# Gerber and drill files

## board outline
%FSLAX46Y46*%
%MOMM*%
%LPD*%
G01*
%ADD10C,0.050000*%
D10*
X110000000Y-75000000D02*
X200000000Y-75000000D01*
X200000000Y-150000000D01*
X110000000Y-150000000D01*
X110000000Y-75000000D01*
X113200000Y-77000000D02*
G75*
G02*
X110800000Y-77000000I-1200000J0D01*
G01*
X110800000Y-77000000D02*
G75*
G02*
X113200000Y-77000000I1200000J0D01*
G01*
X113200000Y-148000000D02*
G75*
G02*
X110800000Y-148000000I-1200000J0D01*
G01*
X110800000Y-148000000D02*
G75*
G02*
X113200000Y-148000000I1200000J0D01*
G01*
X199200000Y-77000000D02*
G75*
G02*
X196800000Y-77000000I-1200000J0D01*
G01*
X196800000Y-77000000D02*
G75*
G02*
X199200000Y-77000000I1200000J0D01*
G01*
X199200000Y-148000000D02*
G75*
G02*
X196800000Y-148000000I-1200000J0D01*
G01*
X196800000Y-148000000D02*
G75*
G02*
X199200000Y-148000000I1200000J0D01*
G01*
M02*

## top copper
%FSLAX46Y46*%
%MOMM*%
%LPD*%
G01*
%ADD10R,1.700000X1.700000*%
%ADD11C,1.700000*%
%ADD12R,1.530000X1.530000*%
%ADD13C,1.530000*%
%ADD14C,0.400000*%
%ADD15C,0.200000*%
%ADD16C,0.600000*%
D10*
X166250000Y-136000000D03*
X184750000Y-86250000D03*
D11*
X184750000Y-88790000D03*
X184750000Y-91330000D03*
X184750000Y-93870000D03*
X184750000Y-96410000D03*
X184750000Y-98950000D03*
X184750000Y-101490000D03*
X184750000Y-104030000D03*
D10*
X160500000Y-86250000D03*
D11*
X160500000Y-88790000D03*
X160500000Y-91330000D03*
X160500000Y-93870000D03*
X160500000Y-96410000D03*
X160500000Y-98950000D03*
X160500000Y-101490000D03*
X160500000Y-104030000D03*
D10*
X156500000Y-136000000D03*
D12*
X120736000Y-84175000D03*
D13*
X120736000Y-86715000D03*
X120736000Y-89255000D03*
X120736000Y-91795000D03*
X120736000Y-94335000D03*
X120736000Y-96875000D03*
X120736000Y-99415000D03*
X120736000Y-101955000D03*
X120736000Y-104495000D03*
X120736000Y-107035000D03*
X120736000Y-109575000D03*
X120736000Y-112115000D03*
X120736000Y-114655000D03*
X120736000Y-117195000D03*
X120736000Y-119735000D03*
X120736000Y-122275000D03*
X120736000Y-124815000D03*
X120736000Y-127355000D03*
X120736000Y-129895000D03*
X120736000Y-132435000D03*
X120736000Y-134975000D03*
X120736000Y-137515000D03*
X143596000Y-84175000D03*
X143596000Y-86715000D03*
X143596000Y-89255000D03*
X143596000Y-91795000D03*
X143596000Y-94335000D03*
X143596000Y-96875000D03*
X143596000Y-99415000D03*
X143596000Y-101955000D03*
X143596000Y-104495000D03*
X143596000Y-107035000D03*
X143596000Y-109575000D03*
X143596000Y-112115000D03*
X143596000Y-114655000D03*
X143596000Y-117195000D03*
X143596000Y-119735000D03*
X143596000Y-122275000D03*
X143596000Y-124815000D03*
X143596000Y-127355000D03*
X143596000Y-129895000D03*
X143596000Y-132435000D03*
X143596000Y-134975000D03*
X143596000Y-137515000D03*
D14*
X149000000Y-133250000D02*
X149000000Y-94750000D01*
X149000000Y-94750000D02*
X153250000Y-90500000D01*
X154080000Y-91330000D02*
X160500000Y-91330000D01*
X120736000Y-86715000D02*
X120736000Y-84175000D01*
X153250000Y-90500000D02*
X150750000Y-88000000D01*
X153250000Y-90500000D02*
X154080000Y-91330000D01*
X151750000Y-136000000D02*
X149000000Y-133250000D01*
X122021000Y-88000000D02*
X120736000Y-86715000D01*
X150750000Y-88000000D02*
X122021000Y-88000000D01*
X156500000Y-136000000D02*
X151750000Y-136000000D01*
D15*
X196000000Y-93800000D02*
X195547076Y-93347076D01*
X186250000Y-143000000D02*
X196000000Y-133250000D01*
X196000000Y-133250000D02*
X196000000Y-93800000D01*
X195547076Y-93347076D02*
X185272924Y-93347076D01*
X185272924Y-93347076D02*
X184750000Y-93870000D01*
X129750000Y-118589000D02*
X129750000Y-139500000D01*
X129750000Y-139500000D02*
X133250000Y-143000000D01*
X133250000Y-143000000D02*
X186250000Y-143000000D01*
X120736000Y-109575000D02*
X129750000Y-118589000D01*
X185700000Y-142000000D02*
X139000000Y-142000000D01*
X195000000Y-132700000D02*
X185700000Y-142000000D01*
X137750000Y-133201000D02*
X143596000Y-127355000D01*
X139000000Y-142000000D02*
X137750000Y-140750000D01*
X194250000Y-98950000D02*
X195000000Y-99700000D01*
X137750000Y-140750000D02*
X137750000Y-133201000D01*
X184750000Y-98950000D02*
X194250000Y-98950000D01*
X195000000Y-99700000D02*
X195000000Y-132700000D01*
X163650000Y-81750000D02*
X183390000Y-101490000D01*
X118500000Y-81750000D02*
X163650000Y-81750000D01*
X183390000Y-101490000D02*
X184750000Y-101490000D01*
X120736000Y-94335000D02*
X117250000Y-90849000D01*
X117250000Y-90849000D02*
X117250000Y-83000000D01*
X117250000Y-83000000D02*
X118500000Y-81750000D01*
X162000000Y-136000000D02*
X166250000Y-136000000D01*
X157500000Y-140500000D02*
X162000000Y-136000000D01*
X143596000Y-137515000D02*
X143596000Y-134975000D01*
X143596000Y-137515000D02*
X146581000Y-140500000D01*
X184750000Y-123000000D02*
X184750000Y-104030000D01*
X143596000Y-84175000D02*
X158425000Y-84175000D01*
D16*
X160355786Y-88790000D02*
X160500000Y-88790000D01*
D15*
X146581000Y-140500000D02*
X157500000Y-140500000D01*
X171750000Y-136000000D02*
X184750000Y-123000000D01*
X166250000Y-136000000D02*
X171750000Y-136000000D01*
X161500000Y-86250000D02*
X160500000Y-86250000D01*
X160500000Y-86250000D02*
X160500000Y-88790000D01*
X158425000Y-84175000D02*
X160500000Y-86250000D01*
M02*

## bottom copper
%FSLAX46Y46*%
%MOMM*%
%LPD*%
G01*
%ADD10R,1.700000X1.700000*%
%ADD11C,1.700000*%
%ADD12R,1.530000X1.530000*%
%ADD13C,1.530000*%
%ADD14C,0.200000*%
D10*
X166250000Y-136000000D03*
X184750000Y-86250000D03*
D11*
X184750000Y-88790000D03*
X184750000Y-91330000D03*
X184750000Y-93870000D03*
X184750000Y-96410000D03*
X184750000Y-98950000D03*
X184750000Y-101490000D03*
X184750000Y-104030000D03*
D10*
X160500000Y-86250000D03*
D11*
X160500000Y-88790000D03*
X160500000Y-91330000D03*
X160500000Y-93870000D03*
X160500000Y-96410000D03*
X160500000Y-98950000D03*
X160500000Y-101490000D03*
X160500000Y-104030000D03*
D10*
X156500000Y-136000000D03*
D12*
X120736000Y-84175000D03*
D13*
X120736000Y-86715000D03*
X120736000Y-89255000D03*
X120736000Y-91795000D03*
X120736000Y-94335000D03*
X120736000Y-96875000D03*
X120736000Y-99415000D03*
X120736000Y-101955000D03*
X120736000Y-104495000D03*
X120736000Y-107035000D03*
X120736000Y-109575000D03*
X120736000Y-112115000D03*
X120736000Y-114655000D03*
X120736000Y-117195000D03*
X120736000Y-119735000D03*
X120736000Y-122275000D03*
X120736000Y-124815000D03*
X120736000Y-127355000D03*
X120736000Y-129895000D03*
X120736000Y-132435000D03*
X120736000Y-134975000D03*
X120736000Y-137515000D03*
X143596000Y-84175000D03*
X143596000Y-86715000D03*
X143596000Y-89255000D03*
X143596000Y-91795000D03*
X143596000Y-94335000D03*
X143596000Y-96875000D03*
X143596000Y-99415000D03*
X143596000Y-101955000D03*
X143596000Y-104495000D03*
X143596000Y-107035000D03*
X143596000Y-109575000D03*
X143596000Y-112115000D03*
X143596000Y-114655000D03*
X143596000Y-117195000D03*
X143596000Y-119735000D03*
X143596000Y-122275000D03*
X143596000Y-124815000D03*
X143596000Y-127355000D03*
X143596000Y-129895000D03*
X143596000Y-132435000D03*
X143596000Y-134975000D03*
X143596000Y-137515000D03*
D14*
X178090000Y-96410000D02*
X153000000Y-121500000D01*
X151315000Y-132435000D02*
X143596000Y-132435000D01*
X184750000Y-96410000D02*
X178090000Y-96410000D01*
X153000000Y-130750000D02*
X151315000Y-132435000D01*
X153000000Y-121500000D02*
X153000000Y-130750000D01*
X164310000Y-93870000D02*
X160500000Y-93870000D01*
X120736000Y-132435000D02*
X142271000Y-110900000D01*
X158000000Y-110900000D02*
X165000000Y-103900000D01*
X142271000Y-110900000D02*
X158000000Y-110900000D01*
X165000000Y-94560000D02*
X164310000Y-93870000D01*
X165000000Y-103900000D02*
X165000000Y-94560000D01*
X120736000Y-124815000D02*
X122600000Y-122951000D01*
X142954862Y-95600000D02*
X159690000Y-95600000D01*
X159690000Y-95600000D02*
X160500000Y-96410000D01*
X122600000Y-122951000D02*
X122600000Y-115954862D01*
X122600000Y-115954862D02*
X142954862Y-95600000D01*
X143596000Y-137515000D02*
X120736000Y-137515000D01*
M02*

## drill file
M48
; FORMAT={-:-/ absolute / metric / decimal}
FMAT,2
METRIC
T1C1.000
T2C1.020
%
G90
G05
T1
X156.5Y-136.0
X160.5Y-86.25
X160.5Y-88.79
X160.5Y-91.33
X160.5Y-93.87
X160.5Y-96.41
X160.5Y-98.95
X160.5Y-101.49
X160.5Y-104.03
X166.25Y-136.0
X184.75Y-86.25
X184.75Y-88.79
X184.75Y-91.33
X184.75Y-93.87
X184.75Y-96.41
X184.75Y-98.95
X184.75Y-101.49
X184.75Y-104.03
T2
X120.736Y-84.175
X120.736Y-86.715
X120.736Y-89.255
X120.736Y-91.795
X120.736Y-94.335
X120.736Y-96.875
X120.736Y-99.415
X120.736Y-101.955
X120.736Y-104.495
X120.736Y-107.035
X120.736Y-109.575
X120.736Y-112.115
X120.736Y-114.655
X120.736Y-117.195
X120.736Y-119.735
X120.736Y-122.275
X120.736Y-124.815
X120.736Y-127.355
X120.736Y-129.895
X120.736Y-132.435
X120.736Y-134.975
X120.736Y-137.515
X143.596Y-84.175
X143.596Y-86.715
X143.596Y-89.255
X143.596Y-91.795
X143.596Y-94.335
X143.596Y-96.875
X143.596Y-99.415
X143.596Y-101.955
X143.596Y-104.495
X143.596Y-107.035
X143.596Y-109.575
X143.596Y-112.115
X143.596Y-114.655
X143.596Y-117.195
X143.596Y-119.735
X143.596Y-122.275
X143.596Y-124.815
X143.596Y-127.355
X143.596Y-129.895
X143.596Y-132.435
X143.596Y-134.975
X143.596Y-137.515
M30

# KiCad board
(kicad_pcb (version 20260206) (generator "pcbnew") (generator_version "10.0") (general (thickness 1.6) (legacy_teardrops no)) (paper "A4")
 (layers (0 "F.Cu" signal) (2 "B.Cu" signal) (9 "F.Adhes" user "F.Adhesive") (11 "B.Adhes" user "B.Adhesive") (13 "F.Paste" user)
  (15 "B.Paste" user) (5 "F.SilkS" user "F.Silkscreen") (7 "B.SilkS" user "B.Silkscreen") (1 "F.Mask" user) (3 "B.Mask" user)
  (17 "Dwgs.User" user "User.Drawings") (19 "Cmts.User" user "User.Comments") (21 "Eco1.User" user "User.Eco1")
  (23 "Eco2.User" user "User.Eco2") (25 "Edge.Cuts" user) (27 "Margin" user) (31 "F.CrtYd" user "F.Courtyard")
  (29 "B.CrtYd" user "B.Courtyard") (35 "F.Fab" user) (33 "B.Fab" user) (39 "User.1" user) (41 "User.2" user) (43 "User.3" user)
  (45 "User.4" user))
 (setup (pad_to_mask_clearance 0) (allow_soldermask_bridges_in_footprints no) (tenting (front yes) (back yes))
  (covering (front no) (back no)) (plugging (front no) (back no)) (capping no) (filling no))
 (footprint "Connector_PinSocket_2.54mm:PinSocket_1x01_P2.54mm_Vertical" (layer "F.Cu") (at 166.25 136 180)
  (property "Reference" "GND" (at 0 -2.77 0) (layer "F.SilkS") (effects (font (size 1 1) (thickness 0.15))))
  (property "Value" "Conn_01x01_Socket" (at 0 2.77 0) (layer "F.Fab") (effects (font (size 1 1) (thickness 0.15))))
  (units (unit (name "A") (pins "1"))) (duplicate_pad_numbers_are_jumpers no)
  (pad "1" thru_hole rect (at 0 0 180) (size 1.7 1.7) (drill 1) (layers "*.Cu" "*.Mask") (remove_unused_layers no) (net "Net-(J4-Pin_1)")))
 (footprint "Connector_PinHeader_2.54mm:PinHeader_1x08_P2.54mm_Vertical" (layer "F.Cu") (at 184.75 86.25)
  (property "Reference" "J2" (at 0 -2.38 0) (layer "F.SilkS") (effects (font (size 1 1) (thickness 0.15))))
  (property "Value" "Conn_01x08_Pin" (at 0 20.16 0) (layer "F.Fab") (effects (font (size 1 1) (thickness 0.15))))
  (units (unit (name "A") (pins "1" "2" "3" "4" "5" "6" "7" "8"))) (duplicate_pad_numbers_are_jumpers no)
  (pad "1" thru_hole rect (at 0 0) (size 1.7 1.7) (drill 1) (layers "*.Cu" "*.Mask") (remove_unused_layers no)
   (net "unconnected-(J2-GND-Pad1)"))
  (pad "2" thru_hole circle (at 0 2.54) (size 1.7 1.7) (drill 1) (layers "*.Cu" "*.Mask") (remove_unused_layers no)
   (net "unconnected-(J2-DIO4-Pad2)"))
  (pad "3" thru_hole circle (at 0 5.08) (size 1.7 1.7) (drill 1) (layers "*.Cu" "*.Mask") (remove_unused_layers no)
   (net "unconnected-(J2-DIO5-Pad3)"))
  (pad "4" thru_hole circle (at 0 7.62) (size 1.7 1.7) (drill 1) (layers "*.Cu" "*.Mask") (remove_unused_layers no) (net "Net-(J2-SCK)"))
  (pad "5" thru_hole circle (at 0 10.16) (size 1.7 1.7) (drill 1) (layers "*.Cu" "*.Mask") (remove_unused_layers no) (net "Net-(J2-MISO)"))
  (pad "6" thru_hole circle (at 0 12.7) (size 1.7 1.7) (drill 1) (layers "*.Cu" "*.Mask") (remove_unused_layers no) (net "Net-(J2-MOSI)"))
  (pad "7" thru_hole circle (at 0 15.24) (size 1.7 1.7) (drill 1) (layers "*.Cu" "*.Mask") (remove_unused_layers no) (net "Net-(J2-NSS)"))
  (pad "8" thru_hole circle (at 0 17.78) (size 1.7 1.7) (drill 1) (layers "*.Cu" "*.Mask") (remove_unused_layers no) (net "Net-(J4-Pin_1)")))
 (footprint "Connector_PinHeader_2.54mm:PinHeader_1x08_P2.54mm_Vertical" (layer "F.Cu") (at 160.5 86.25)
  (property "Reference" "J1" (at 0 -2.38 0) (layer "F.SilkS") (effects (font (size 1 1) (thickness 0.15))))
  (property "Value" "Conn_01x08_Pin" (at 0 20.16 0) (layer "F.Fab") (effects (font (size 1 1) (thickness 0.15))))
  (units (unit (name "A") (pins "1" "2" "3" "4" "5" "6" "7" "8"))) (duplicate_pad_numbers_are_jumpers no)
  (pad "1" thru_hole rect (at 0 0) (size 1.7 1.7) (drill 1) (layers "*.Cu" "*.Mask") (remove_unused_layers no) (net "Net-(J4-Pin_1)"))
  (pad "2" thru_hole circle (at 0 2.54) (size 1.7 1.7) (drill 1) (layers "*.Cu" "*.Mask") (remove_unused_layers no) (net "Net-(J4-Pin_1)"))
  (pad "3" thru_hole circle (at 0 5.08) (size 1.7 1.7) (drill 1) (layers "*.Cu" "*.Mask") (remove_unused_layers no) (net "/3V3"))
  (pad "4" thru_hole circle (at 0 7.62) (size 1.7 1.7) (drill 1) (layers "*.Cu" "*.Mask") (remove_unused_layers no) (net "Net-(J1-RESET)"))
  (pad "5" thru_hole circle (at 0 10.16) (size 1.7 1.7) (drill 1) (layers "*.Cu" "*.Mask") (remove_unused_layers no) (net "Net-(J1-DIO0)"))
  (pad "6" thru_hole circle (at 0 12.7) (size 1.7 1.7) (drill 1) (layers "*.Cu" "*.Mask") (remove_unused_layers no)
   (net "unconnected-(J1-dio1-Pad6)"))
  (pad "7" thru_hole circle (at 0 15.24) (size 1.7 1.7) (drill 1) (layers "*.Cu" "*.Mask") (remove_unused_layers no)
   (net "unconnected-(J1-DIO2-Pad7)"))
  (pad "8" thru_hole circle (at 0 17.78) (size 1.7 1.7) (drill 1) (layers "*.Cu" "*.Mask") (remove_unused_layers no)
   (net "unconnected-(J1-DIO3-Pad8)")))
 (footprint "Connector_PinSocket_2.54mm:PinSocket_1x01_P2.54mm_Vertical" (layer "F.Cu") (at 156.5 136 180)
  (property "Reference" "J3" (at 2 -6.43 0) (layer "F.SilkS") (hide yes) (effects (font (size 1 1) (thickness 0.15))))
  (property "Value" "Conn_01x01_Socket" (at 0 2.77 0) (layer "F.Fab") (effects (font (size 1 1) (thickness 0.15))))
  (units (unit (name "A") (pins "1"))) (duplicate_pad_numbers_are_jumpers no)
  (pad "1" thru_hole rect (at 0 0 180) (size 1.7 1.7) (drill 1) (layers "*.Cu" "*.Mask") (remove_unused_layers no) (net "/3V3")))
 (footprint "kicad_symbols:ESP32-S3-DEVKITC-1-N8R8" (layer "F.Cu") (at 132.166 114.145)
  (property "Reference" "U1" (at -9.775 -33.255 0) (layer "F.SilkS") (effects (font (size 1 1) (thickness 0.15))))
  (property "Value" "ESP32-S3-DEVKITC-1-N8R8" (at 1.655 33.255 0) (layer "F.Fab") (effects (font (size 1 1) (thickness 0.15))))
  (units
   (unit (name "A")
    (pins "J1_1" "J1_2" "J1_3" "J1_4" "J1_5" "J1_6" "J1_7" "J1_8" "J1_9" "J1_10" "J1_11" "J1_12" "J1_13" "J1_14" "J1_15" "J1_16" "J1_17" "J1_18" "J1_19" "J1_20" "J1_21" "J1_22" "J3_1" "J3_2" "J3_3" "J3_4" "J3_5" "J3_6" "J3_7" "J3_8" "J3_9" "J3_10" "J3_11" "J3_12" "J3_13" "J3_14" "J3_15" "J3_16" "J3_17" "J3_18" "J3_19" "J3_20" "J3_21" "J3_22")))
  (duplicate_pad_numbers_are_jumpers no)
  (pad "J1_1" thru_hole rect (at -11.43 -29.97) (size 1.53 1.53) (drill 1.02) (layers "*.Cu" "*.Mask") (remove_unused_layers no)
   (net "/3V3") (solder_mask_margin 0.102))
  (pad "J1_2" thru_hole circle (at -11.43 -27.43) (size 1.53 1.53) (drill 1.02) (layers "*.Cu" "*.Mask") (remove_unused_layers no)
   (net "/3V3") (solder_mask_margin 0.102))
  (pad "J1_3" thru_hole circle (at -11.43 -24.89) (size 1.53 1.53) (drill 1.02) (layers "*.Cu" "*.Mask") (remove_unused_layers no)
   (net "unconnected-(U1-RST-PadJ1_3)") (solder_mask_margin 0.102))
  (pad "J1_4" thru_hole circle (at -11.43 -22.35) (size 1.53 1.53) (drill 1.02) (layers "*.Cu" "*.Mask") (remove_unused_layers no)
   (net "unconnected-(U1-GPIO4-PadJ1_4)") (solder_mask_margin 0.102))
  (pad "J1_5" thru_hole circle (at -11.43 -19.81) (size 1.53 1.53) (drill 1.02) (layers "*.Cu" "*.Mask") (remove_unused_layers no)
   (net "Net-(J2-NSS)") (solder_mask_margin 0.102))
  (pad "J1_6" thru_hole circle (at -11.43 -17.27) (size 1.53 1.53) (drill 1.02) (layers "*.Cu" "*.Mask") (remove_unused_layers no)
   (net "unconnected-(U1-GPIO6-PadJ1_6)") (solder_mask_margin 0.102))
  (pad "J1_7" thru_hole circle (at -11.43 -14.73) (size 1.53 1.53) (drill 1.02) (layers "*.Cu" "*.Mask") (remove_unused_layers no)
   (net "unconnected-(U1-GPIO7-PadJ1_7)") (solder_mask_margin 0.102))
  (pad "J1_8" thru_hole circle (at -11.43 -12.19) (size 1.53 1.53) (drill 1.02) (layers "*.Cu" "*.Mask") (remove_unused_layers no)
   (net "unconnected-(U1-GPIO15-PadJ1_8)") (solder_mask_margin 0.102))
  (pad "J1_9" thru_hole circle (at -11.43 -9.65) (size 1.53 1.53) (drill 1.02) (layers "*.Cu" "*.Mask") (remove_unused_layers no)
   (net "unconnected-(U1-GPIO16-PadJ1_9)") (solder_mask_margin 0.102))
  (pad "J1_10" thru_hole circle (at -11.43 -7.11) (size 1.53 1.53) (drill 1.02) (layers "*.Cu" "*.Mask") (remove_unused_layers no)
   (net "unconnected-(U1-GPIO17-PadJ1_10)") (solder_mask_margin 0.102))
  (pad "J1_11" thru_hole circle (at -11.43 -4.57) (size 1.53 1.53) (drill 1.02) (layers "*.Cu" "*.Mask") (remove_unused_layers no)
   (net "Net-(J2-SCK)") (solder_mask_margin 0.102))
  (pad "J1_12" thru_hole circle (at -11.43 -2.03) (size 1.53 1.53) (drill 1.02) (layers "*.Cu" "*.Mask") (remove_unused_layers no)
   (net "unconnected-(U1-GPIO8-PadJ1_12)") (solder_mask_margin 0.102))
  (pad "J1_13" thru_hole circle (at -11.43 0.51) (size 1.53 1.53) (drill 1.02) (layers "*.Cu" "*.Mask") (remove_unused_layers no)
   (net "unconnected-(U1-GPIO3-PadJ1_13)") (solder_mask_margin 0.102))
  (pad "J1_14" thru_hole circle (at -11.43 3.05) (size 1.53 1.53) (drill 1.02) (layers "*.Cu" "*.Mask") (remove_unused_layers no)
   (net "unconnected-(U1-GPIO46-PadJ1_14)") (solder_mask_margin 0.102))
  (pad "J1_15" thru_hole circle (at -11.43 5.59) (size 1.53 1.53) (drill 1.02) (layers "*.Cu" "*.Mask") (remove_unused_layers no)
   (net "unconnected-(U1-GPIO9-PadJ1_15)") (solder_mask_margin 0.102))
  (pad "J1_16" thru_hole circle (at -11.43 8.13) (size 1.53 1.53) (drill 1.02) (layers "*.Cu" "*.Mask") (remove_unused_layers no)
   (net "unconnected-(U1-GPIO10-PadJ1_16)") (solder_mask_margin 0.102))
  (pad "J1_17" thru_hole circle (at -11.43 10.67) (size 1.53 1.53) (drill 1.02) (layers "*.Cu" "*.Mask") (remove_unused_layers no)
   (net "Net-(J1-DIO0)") (solder_mask_margin 0.102))
  (pad "J1_18" thru_hole circle (at -11.43 13.21) (size 1.53 1.53) (drill 1.02) (layers "*.Cu" "*.Mask") (remove_unused_layers no)
   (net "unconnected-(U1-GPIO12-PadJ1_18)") (solder_mask_margin 0.102))
  (pad "J1_19" thru_hole circle (at -11.43 15.75) (size 1.53 1.53) (drill 1.02) (layers "*.Cu" "*.Mask") (remove_unused_layers no)
   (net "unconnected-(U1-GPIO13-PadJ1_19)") (solder_mask_margin 0.102))
  (pad "J1_20" thru_hole circle (at -11.43 18.29) (size 1.53 1.53) (drill 1.02) (layers "*.Cu" "*.Mask") (remove_unused_layers no)
   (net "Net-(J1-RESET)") (solder_mask_margin 0.102))
  (pad "J1_21" thru_hole circle (at -11.43 20.83) (size 1.53 1.53) (drill 1.02) (layers "*.Cu" "*.Mask") (remove_unused_layers no)
   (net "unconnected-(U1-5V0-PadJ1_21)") (solder_mask_margin 0.102))
  (pad "J1_22" thru_hole circle (at -11.43 23.37) (size 1.53 1.53) (drill 1.02) (layers "*.Cu" "*.Mask") (remove_unused_layers no)
   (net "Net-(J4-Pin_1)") (solder_mask_margin 0.102))
  (pad "J3_1" thru_hole circle (at 11.43 -29.97) (size 1.53 1.53) (drill 1.02) (layers "*.Cu" "*.Mask") (remove_unused_layers no)
   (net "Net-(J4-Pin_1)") (solder_mask_margin 0.102))
  (pad "J3_2" thru_hole circle (at 11.43 -27.43) (size 1.53 1.53) (drill 1.02) (layers "*.Cu" "*.Mask") (remove_unused_layers no)
   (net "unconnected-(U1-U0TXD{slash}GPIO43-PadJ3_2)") (solder_mask_margin 0.102))
  (pad "J3_3" thru_hole circle (at 11.43 -24.89) (size 1.53 1.53) (drill 1.02) (layers "*.Cu" "*.Mask") (remove_unused_layers no)
   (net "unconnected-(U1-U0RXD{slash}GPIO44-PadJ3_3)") (solder_mask_margin 0.102))
  (pad "J3_4" thru_hole circle (at 11.43 -22.35) (size 1.53 1.53) (drill 1.02) (layers "*.Cu" "*.Mask") (remove_unused_layers no)
   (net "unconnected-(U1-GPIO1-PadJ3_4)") (solder_mask_margin 0.102))
  (pad "J3_5" thru_hole circle (at 11.43 -19.81) (size 1.53 1.53) (drill 1.02) (layers "*.Cu" "*.Mask") (remove_unused_layers no)
   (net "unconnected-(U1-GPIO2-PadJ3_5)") (solder_mask_margin 0.102))
  (pad "J3_6" thru_hole circle (at 11.43 -17.27) (size 1.53 1.53) (drill 1.02) (layers "*.Cu" "*.Mask") (remove_unused_layers no)
   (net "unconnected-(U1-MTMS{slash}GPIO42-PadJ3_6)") (solder_mask_margin 0.102))
  (pad "J3_7" thru_hole circle (at 11.43 -14.73) (size 1.53 1.53) (drill 1.02) (layers "*.Cu" "*.Mask") (remove_unused_layers no)
   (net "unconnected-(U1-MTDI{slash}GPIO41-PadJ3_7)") (solder_mask_margin 0.102))
  (pad "J3_8" thru_hole circle (at 11.43 -12.19) (size 1.53 1.53) (drill 1.02) (layers "*.Cu" "*.Mask") (remove_unused_layers no)
   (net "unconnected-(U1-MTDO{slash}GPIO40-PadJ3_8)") (solder_mask_margin 0.102))
  (pad "J3_9" thru_hole circle (at 11.43 -9.65) (size 1.53 1.53) (drill 1.02) (layers "*.Cu" "*.Mask") (remove_unused_layers no)
   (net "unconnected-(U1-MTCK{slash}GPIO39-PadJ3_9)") (solder_mask_margin 0.102))
  (pad "J3_10" thru_hole circle (at 11.43 -7.11) (size 1.53 1.53) (drill 1.02) (layers "*.Cu" "*.Mask") (remove_unused_layers no)
   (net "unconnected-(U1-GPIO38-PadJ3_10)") (solder_mask_margin 0.102))
  (pad "J3_11" thru_hole circle (at 11.43 -4.57) (size 1.53 1.53) (drill 1.02) (layers "*.Cu" "*.Mask") (remove_unused_layers no)
   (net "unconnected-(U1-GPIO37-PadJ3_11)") (solder_mask_margin 0.102))
  (pad "J3_12" thru_hole circle (at 11.43 -2.03) (size 1.53 1.53) (drill 1.02) (layers "*.Cu" "*.Mask") (remove_unused_layers no)
   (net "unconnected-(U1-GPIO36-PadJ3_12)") (solder_mask_margin 0.102))
  (pad "J3_13" thru_hole circle (at 11.43 0.51) (size 1.53 1.53) (drill 1.02) (layers "*.Cu" "*.Mask") (remove_unused_layers no)
   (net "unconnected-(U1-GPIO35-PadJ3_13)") (solder_mask_margin 0.102))
  (pad "J3_14" thru_hole circle (at 11.43 3.05) (size 1.53 1.53) (drill 1.02) (layers "*.Cu" "*.Mask") (remove_unused_layers no)
   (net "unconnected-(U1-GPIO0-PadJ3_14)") (solder_mask_margin 0.102))
  (pad "J3_15" thru_hole circle (at 11.43 5.59) (size 1.53 1.53) (drill 1.02) (layers "*.Cu" "*.Mask") (remove_unused_layers no)
   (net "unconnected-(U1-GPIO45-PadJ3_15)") (solder_mask_margin 0.102))
  (pad "J3_16" thru_hole circle (at 11.43 8.13) (size 1.53 1.53) (drill 1.02) (layers "*.Cu" "*.Mask") (remove_unused_layers no)
   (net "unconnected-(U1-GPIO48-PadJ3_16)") (solder_mask_margin 0.102))
  (pad "J3_17" thru_hole circle (at 11.43 10.67) (size 1.53 1.53) (drill 1.02) (layers "*.Cu" "*.Mask") (remove_unused_layers no)
   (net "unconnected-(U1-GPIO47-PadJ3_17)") (solder_mask_margin 0.102))
  (pad "J3_18" thru_hole circle (at 11.43 13.21) (size 1.53 1.53) (drill 1.02) (layers "*.Cu" "*.Mask") (remove_unused_layers no)
   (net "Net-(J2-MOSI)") (solder_mask_margin 0.102))
  (pad "J3_19" thru_hole circle (at 11.43 15.75) (size 1.53 1.53) (drill 1.02) (layers "*.Cu" "*.Mask") (remove_unused_layers no)
   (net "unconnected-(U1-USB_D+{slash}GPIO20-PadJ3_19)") (solder_mask_margin 0.102))
  (pad "J3_20" thru_hole circle (at 11.43 18.29) (size 1.53 1.53) (drill 1.02) (layers "*.Cu" "*.Mask") (remove_unused_layers no)
   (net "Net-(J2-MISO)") (solder_mask_margin 0.102))
  (pad "J3_21" thru_hole circle (at 11.43 20.83) (size 1.53 1.53) (drill 1.02) (layers "*.Cu" "*.Mask") (remove_unused_layers no)
   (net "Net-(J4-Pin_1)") (solder_mask_margin 0.102))
  (pad "J3_22" thru_hole circle (at 11.43 23.37) (size 1.53 1.53) (drill 1.02) (layers "*.Cu" "*.Mask") (remove_unused_layers no)
   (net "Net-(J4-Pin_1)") (solder_mask_margin 0.102)))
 (gr_rect (start 110 75) (end 200 150) (stroke (width 0.05) (type solid)) (fill no) (layer "Edge.Cuts"))
 (gr_circle (center 112 77) (end 113.2 77) (stroke (width 0.05) (type default)) (fill no) (layer "Edge.Cuts"))
 (gr_circle (center 112 148) (end 113.2 148) (stroke (width 0.05) (type default)) (fill no) (layer "Edge.Cuts"))
 (gr_circle (center 198 77) (end 199.2 77) (stroke (width 0.05) (type default)) (fill no) (layer "Edge.Cuts"))
 (gr_circle (center 198 148) (end 199.2 148) (stroke (width 0.05) (type default)) (fill no) (layer "Edge.Cuts"))
 (segment (start 149 133.25) (end 149 94.75) (width 0.4) (layer "F.Cu") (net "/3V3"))
 (segment (start 149 94.75) (end 153.25 90.5) (width 0.4) (layer "F.Cu") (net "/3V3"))
 (segment (start 154.08 91.33) (end 160.5 91.33) (width 0.4) (layer "F.Cu") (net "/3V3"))
 (segment (start 120.736 86.715) (end 120.736 84.175) (width 0.4) (layer "F.Cu") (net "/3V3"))
 (segment (start 153.25 90.5) (end 150.75 88) (width 0.4) (layer "F.Cu") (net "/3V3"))
 (segment (start 153.25 90.5) (end 154.08 91.33) (width 0.4) (layer "F.Cu") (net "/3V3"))
 (segment (start 151.75 136) (end 149 133.25) (width 0.4) (layer "F.Cu") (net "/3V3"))
 (segment (start 122.021 88) (end 120.736 86.715) (width 0.4) (layer "F.Cu") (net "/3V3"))
 (segment (start 150.75 88) (end 122.021 88) (width 0.4) (layer "F.Cu") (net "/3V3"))
 (segment (start 156.5 136) (end 151.75 136) (width 0.4) (layer "F.Cu") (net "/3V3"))
 (segment (start 196 93.8) (end 195.547076 93.347076) (width 0.2) (layer "F.Cu") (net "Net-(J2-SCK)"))
 (segment (start 186.25 143) (end 196 133.25) (width 0.2) (layer "F.Cu") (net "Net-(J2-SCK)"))
 (segment (start 196 133.25) (end 196 93.8) (width 0.2) (layer "F.Cu") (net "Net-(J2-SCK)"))
 (segment (start 195.547076 93.347076) (end 185.272924 93.347076) (width 0.2) (layer "F.Cu") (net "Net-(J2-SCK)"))
 (segment (start 185.272924 93.347076) (end 184.75 93.87) (width 0.2) (layer "F.Cu") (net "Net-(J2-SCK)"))
 (segment (start 129.75 118.589) (end 129.75 139.5) (width 0.2) (layer "F.Cu") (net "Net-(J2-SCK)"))
 (segment (start 129.75 139.5) (end 133.25 143) (width 0.2) (layer "F.Cu") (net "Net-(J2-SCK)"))
 (segment (start 133.25 143) (end 186.25 143) (width 0.2) (layer "F.Cu") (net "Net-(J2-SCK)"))
 (segment (start 120.736 109.575) (end 129.75 118.589) (width 0.2) (layer "F.Cu") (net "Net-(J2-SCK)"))
 (segment (start 178.09 96.41) (end 153 121.5) (width 0.2) (layer "B.Cu") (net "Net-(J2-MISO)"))
 (segment (start 151.315 132.435) (end 143.596 132.435) (width 0.2) (layer "B.Cu") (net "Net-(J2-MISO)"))
 (segment (start 184.75 96.41) (end 178.09 96.41) (width 0.2) (layer "B.Cu") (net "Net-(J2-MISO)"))
 (segment (start 153 130.75) (end 151.315 132.435) (width 0.2) (layer "B.Cu") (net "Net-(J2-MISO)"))
 (segment (start 153 121.5) (end 153 130.75) (width 0.2) (layer "B.Cu") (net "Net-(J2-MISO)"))
 (segment (start 185.7 142) (end 139 142) (width 0.2) (layer "F.Cu") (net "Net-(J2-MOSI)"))
 (segment (start 195 132.7) (end 185.7 142) (width 0.2) (layer "F.Cu") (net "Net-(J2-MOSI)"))
 (segment (start 137.75 133.201) (end 143.596 127.355) (width 0.2) (layer "F.Cu") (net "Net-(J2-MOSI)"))
 (segment (start 139 142) (end 137.75 140.75) (width 0.2) (layer "F.Cu") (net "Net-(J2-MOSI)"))
 (segment (start 194.25 98.95) (end 195 99.7) (width 0.2) (layer "F.Cu") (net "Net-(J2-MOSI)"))
 (segment (start 137.75 140.75) (end 137.75 133.201) (width 0.2) (layer "F.Cu") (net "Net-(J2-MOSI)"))
 (segment (start 184.75 98.95) (end 194.25 98.95) (width 0.2) (layer "F.Cu") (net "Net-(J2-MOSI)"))
 (segment (start 195 99.7) (end 195 132.7) (width 0.2) (layer "F.Cu") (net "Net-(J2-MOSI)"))
 (segment (start 163.65 81.75) (end 183.39 101.49) (width 0.2) (layer "F.Cu") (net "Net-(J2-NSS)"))
 (segment (start 118.5 81.75) (end 163.65 81.75) (width 0.2) (layer "F.Cu") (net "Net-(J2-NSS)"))
 (segment (start 183.39 101.49) (end 184.75 101.49) (width 0.2) (layer "F.Cu") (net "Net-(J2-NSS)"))
 (segment (start 120.736 94.335) (end 117.25 90.849) (width 0.2) (layer "F.Cu") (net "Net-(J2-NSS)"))
 (segment (start 117.25 90.849) (end 117.25 83) (width 0.2) (layer "F.Cu") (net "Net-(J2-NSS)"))
 (segment (start 117.25 83) (end 118.5 81.75) (width 0.2) (layer "F.Cu") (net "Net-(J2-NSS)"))
 (segment (start 164.31 93.87) (end 160.5 93.87) (width 0.2) (layer "B.Cu") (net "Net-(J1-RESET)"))
 (segment (start 120.736 132.435) (end 142.271 110.9) (width 0.2) (layer "B.Cu") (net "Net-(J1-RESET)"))
 (segment (start 158 110.9) (end 165 103.9) (width 0.2) (layer "B.Cu") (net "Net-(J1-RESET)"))
 (segment (start 142.271 110.9) (end 158 110.9) (width 0.2) (layer "B.Cu") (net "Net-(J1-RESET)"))
 (segment (start 165 94.56) (end 164.31 93.87) (width 0.2) (layer "B.Cu") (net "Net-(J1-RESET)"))
 (segment (start 165 103.9) (end 165 94.56) (width 0.2) (layer "B.Cu") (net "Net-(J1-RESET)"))
 (segment (start 120.736 124.815) (end 122.6 122.951) (width 0.2) (layer "B.Cu") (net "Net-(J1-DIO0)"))
 (segment (start 142.954862 95.6) (end 159.69 95.6) (width 0.2) (layer "B.Cu") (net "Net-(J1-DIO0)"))
 (segment (start 159.69 95.6) (end 160.5 96.41) (width 0.2) (layer "B.Cu") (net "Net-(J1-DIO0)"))
 (segment (start 122.6 122.951) (end 122.6 115.954862) (width 0.2) (layer "B.Cu") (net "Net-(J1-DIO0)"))
 (segment (start 122.6 115.954862) (end 142.954862 95.6) (width 0.2) (layer "B.Cu") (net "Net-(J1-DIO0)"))
 (segment (start 162 136) (end 166.25 136) (width 0.2) (layer "F.Cu") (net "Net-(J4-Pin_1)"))
 (segment (start 157.5 140.5) (end 162 136) (width 0.2) (layer "F.Cu") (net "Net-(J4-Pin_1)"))
 (segment (start 143.596 137.515) (end 143.596 134.975) (width 0.2) (layer "F.Cu") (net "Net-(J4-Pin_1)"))
 (segment (start 143.596 137.515) (end 146.581 140.5) (width 0.2) (layer "F.Cu") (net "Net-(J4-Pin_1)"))
 (segment (start 184.75 123) (end 184.75 104.03) (width 0.2) (layer "F.Cu") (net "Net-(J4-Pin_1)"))
 (segment (start 143.596 84.175) (end 158.425 84.175) (width 0.2) (layer "F.Cu") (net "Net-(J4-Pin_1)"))
 (segment (start 160.355786 88.79) (end 160.5 88.79) (width 0.6) (layer "F.Cu") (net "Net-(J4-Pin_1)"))
 (segment (start 146.581 140.5) (end 157.5 140.5) (width 0.2) (layer "F.Cu") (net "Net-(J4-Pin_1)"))
 (segment (start 171.75 136) (end 184.75 123) (width 0.2) (layer "F.Cu") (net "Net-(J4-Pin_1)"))
 (segment (start 166.25 136) (end 171.75 136) (width 0.2) (layer "F.Cu") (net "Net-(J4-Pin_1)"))
 (segment (start 161.5 86.25) (end 160.5 86.25) (width 0.2) (layer "F.Cu") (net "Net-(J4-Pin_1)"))
 (segment (start 160.5 86.25) (end 160.5 88.79) (width 0.2) (layer "F.Cu") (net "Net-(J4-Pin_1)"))
 (segment (start 158.425 84.175) (end 160.5 86.25) (width 0.2) (layer "F.Cu") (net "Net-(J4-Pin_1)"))
 (segment (start 143.596 137.515) (end 120.736 137.515) (width 0.2) (layer "B.Cu") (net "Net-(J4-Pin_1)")))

